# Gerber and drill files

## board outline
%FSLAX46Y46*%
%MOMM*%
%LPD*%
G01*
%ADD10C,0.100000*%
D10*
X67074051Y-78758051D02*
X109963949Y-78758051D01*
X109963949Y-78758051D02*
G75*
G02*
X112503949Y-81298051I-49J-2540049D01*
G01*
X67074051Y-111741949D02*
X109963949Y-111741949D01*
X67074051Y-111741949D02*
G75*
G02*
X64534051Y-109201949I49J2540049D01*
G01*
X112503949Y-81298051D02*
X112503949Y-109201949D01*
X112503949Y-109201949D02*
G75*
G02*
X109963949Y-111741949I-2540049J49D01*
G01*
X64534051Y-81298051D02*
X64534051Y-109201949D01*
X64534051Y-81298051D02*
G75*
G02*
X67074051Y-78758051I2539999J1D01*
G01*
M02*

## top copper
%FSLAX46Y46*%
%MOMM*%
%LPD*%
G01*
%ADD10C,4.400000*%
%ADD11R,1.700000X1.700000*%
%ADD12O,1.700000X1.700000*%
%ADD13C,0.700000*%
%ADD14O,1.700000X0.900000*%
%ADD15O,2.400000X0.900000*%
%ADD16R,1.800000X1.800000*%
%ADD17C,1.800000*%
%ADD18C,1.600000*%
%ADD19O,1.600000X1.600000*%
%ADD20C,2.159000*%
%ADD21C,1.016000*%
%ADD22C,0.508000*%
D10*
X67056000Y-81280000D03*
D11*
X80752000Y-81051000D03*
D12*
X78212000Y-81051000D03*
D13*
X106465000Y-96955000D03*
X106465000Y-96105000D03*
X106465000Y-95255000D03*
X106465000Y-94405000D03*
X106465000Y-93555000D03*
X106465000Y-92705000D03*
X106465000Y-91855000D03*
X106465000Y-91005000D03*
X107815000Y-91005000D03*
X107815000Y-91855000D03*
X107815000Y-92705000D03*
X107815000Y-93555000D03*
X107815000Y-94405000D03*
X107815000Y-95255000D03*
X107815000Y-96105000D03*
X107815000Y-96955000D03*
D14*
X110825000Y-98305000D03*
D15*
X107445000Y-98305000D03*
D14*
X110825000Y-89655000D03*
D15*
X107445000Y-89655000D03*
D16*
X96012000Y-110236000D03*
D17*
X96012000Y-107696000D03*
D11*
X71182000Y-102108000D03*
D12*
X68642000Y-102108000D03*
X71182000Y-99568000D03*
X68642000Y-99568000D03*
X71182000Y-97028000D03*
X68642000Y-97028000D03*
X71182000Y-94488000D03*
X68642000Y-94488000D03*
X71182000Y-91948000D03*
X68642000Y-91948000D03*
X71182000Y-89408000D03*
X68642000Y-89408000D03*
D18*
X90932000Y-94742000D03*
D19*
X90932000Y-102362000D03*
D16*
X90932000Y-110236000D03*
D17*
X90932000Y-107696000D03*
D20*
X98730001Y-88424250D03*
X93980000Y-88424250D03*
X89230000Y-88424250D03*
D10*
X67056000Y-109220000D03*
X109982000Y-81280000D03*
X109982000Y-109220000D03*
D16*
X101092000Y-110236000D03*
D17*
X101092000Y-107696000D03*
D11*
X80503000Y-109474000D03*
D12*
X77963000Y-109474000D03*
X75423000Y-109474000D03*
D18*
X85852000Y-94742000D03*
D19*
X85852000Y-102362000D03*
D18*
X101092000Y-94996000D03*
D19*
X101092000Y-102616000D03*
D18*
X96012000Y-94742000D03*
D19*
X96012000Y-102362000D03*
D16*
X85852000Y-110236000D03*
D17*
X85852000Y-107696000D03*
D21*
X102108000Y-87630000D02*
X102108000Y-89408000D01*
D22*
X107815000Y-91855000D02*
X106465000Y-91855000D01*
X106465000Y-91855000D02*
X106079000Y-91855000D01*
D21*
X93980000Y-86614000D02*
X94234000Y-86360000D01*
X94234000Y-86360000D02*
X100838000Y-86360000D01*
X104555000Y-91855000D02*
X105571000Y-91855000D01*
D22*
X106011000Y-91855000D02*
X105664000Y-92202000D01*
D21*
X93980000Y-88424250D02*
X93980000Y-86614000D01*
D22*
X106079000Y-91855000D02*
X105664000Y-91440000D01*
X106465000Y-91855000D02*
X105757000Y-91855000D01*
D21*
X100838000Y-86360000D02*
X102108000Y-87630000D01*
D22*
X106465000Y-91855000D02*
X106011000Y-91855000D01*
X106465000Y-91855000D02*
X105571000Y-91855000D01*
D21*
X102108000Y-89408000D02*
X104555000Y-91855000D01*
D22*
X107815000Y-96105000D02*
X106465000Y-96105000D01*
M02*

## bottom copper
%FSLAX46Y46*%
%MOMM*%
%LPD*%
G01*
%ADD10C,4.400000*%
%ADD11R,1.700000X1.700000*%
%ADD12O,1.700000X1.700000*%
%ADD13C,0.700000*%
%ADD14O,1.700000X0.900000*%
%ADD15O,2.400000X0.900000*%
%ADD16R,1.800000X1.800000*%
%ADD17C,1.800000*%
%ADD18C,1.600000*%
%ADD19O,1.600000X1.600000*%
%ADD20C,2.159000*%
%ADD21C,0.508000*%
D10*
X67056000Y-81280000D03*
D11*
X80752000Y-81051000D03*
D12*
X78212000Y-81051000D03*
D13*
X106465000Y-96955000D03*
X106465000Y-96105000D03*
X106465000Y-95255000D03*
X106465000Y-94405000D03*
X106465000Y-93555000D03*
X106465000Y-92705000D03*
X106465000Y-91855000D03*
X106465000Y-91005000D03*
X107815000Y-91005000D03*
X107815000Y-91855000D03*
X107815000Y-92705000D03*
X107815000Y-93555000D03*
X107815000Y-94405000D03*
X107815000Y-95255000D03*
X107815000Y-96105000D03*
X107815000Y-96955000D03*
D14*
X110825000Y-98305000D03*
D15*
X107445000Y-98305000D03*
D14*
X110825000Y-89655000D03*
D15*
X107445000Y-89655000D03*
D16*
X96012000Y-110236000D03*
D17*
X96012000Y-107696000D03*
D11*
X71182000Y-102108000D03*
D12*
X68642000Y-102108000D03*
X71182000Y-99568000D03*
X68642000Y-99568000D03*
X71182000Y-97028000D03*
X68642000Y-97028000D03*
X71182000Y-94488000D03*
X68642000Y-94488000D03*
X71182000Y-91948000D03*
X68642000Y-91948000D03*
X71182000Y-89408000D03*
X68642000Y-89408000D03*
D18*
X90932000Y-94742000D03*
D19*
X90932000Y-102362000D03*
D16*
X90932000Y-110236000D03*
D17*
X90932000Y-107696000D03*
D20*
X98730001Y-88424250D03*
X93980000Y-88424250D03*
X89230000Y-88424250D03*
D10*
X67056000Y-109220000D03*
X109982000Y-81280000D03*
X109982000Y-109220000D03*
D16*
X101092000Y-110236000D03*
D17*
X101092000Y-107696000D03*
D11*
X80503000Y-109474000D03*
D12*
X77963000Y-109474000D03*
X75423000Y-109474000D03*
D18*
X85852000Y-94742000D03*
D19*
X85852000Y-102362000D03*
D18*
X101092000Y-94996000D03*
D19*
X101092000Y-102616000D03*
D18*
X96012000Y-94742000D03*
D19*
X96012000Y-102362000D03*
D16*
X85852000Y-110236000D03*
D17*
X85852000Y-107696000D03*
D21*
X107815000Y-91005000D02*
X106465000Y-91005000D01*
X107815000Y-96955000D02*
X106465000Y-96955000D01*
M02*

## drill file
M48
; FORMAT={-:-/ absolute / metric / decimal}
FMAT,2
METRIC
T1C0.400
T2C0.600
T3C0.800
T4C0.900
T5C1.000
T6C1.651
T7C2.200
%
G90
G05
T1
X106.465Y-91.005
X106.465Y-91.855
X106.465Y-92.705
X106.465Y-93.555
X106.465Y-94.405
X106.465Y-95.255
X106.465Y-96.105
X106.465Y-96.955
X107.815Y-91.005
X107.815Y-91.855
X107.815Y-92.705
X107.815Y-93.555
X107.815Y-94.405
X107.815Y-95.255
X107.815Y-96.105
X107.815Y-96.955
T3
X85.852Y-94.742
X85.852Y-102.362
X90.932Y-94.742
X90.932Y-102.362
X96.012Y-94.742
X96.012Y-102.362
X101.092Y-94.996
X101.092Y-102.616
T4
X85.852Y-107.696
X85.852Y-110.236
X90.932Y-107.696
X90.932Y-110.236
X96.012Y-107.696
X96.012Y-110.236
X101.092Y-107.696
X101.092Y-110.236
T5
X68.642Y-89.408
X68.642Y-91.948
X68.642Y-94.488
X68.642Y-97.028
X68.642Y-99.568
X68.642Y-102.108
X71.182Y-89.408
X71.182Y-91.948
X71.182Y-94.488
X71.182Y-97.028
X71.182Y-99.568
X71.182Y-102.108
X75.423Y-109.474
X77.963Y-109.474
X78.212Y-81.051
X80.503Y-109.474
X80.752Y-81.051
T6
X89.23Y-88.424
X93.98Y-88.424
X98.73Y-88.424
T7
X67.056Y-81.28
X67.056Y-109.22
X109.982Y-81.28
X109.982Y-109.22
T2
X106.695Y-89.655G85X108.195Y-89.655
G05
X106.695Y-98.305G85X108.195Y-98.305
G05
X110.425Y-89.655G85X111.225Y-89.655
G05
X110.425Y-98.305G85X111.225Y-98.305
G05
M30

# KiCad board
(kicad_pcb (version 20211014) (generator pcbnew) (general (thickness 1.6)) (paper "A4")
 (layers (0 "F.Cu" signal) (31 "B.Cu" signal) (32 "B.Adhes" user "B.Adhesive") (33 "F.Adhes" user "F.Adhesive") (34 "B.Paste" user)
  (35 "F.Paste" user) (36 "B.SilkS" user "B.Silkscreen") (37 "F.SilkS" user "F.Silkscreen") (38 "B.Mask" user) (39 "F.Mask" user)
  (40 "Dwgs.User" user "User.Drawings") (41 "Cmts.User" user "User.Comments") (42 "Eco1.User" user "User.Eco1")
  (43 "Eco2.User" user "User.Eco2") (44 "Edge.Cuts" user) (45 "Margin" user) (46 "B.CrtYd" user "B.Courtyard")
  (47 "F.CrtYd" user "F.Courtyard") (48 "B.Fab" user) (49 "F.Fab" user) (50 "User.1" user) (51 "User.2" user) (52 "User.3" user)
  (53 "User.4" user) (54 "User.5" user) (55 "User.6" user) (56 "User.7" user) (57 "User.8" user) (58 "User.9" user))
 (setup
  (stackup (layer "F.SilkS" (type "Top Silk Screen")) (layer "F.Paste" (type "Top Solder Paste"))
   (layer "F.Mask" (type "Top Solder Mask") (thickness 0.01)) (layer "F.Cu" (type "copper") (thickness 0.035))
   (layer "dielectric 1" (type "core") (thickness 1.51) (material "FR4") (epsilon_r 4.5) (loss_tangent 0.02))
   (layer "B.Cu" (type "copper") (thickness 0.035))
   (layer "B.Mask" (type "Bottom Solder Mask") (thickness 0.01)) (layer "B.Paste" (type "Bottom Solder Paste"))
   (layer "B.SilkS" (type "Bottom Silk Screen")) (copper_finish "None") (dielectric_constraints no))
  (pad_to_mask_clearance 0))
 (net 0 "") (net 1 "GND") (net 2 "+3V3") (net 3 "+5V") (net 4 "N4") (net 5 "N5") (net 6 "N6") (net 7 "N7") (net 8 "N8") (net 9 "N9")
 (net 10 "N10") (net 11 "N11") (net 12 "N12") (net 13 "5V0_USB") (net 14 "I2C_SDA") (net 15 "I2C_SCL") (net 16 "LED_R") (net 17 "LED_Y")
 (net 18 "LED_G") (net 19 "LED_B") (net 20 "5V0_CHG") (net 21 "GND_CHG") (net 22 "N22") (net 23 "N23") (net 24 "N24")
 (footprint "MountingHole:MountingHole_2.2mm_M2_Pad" (layer "F.Cu") (at 67.056 81.28)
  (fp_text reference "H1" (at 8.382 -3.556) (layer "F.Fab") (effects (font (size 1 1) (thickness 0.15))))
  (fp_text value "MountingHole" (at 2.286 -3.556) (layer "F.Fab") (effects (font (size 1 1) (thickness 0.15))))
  (pad "1" thru_hole circle (at 0 0) (size 4.4 4.4) (drill 2.2) (layers *.Cu *.Mask)))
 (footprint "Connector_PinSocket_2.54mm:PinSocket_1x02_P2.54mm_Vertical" (layer "F.Cu") (at 80.752 81.051 -90)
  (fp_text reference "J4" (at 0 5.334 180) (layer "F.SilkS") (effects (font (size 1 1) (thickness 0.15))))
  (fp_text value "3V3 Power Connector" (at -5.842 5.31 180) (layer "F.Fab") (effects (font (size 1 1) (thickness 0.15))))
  (pad "1" thru_hole rect (at 0 0 270) (size 1.7 1.7) (drill 1) (layers *.Cu *.Mask) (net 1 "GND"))
  (pad "2" thru_hole oval (at 0 2.54 270) (size 1.7 1.7) (drill 1) (layers *.Cu *.Mask) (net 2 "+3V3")))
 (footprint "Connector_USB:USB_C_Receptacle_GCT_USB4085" (layer "F.Cu") (at 106.465 96.955 90)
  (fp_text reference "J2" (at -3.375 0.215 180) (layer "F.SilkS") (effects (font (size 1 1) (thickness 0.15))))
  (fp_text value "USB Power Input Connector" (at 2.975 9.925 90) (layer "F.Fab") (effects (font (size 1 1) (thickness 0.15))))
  (pad "A1" thru_hole circle (at 0 0 90) (size 0.7 0.7) (drill 0.4) (layers *.Cu *.Mask) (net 1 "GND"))
  (pad "A4" thru_hole circle (at 0.85 0 90) (size 0.7 0.7) (drill 0.4) (layers *.Cu *.Mask) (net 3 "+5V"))
  (pad "A5" thru_hole circle (at 1.7 0 90) (size 0.7 0.7) (drill 0.4) (layers *.Cu *.Mask) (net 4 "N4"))
  (pad "A6" thru_hole circle (at 2.55 0 90) (size 0.7 0.7) (drill 0.4) (layers *.Cu *.Mask) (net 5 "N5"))
  (pad "A7" thru_hole circle (at 3.4 0 90) (size 0.7 0.7) (drill 0.4) (layers *.Cu *.Mask) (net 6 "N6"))
  (pad "A8" thru_hole circle (at 4.25 0 90) (size 0.7 0.7) (drill 0.4) (layers *.Cu *.Mask) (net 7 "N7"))
  (pad "A9" thru_hole circle (at 5.1 0 90) (size 0.7 0.7) (drill 0.4) (layers *.Cu *.Mask) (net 3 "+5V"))
  (pad "A12" thru_hole circle (at 5.95 0 90) (size 0.7 0.7) (drill 0.4) (layers *.Cu *.Mask) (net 1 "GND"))
  (pad "B1" thru_hole circle (at 5.95 1.35 90) (size 0.7 0.7) (drill 0.4) (layers *.Cu *.Mask) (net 1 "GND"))
  (pad "B4" thru_hole circle (at 5.1 1.35 90) (size 0.7 0.7) (drill 0.4) (layers *.Cu *.Mask) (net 3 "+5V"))
  (pad "B5" thru_hole circle (at 4.25 1.35 90) (size 0.7 0.7) (drill 0.4) (layers *.Cu *.Mask) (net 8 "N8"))
  (pad "B6" thru_hole circle (at 3.4 1.35 90) (size 0.7 0.7) (drill 0.4) (layers *.Cu *.Mask) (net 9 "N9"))
  (pad "B7" thru_hole circle (at 2.55 1.35 90) (size 0.7 0.7) (drill 0.4) (layers *.Cu *.Mask) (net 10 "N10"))
  (pad "B8" thru_hole circle (at 1.7 1.35 90) (size 0.7 0.7) (drill 0.4) (layers *.Cu *.Mask) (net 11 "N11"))
  (pad "B9" thru_hole circle (at 0.85 1.35 90) (size 0.7 0.7) (drill 0.4) (layers *.Cu *.Mask) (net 3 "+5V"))
  (pad "B12" thru_hole circle (at 0 1.35 90) (size 0.7 0.7) (drill 0.4) (layers *.Cu *.Mask) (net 1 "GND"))
  (pad "S1" thru_hole oval (at -1.35 4.36 90) (size 0.9 1.7) (drill oval 0.6 1.4) (layers *.Cu *.Mask) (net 1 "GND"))
  (pad "S1" thru_hole oval (at -1.35 0.98 90) (size 0.9 2.4) (drill oval 0.6 2.1) (layers *.Cu *.Mask) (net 1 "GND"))
  (pad "S1" thru_hole oval (at 7.3 4.36 90) (size 0.9 1.7) (drill oval 0.6 1.4) (layers *.Cu *.Mask) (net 1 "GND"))
  (pad "S1" thru_hole oval (at 7.3 0.98 90) (size 0.9 2.4) (drill oval 0.6 2.1) (layers *.Cu *.Mask) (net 1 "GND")))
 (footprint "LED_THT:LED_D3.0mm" (layer "F.Cu") (at 96.012 110.236 90)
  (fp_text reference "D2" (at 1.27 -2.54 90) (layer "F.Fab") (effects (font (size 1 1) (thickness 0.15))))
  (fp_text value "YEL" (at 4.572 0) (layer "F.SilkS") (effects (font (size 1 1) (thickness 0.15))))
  (pad "1" thru_hole rect (at 0 0 90) (size 1.8 1.8) (drill 0.9) (layers *.Cu *.Mask) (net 1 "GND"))
  (pad "2" thru_hole circle (at 2.54 0 90) (size 1.8 1.8) (drill 0.9) (layers *.Cu *.Mask) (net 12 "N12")))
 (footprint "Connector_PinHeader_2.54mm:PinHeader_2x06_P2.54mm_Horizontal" (layer "F.Cu") (at 71.182 102.108 180)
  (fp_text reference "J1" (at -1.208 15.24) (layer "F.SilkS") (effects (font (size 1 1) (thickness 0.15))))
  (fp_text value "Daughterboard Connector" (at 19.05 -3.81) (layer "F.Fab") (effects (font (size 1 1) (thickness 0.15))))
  (pad "1" thru_hole rect (at 0 0 180) (size 1.7 1.7) (drill 1) (layers *.Cu *.Mask) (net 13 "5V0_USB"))
  (pad "2" thru_hole oval (at 2.54 0 180) (size 1.7 1.7) (drill 1) (layers *.Cu *.Mask) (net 2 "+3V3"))
  (pad "3" thru_hole oval (at 0 2.54 180) (size 1.7 1.7) (drill 1) (layers *.Cu *.Mask) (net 1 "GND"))
  (pad "4" thru_hole oval (at 2.54 2.54 180) (size 1.7 1.7) (drill 1) (layers *.Cu *.Mask) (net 1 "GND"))
  (pad "5" thru_hole oval (at 0 5.08 180) (size 1.7 1.7) (drill 1) (layers *.Cu *.Mask) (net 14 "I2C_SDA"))
  (pad "6" thru_hole oval (at 2.54 5.08 180) (size 1.7 1.7) (drill 1) (layers *.Cu *.Mask) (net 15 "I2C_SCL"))
  (pad "7" thru_hole oval (at 0 7.62 180) (size 1.7 1.7) (drill 1) (layers *.Cu *.Mask) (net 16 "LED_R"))
  (pad "8" thru_hole oval (at 2.54 7.62 180) (size 1.7 1.7) (drill 1) (layers *.Cu *.Mask) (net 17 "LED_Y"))
  (pad "9" thru_hole oval (at 0 10.16 180) (size 1.7 1.7) (drill 1) (layers *.Cu *.Mask) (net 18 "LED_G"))
  (pad "10" thru_hole oval (at 2.54 10.16 180) (size 1.7 1.7) (drill 1) (layers *.Cu *.Mask) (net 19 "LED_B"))
  (pad "11" thru_hole oval (at 0 12.7 180) (size 1.7 1.7) (drill 1) (layers *.Cu *.Mask) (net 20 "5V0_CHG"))
  (pad "12" thru_hole oval (at 2.54 12.7 180) (size 1.7 1.7) (drill 1) (layers *.Cu *.Mask) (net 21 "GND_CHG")))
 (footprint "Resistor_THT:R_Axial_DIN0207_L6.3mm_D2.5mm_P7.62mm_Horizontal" (layer "F.Cu") (at 90.932 94.742 -90)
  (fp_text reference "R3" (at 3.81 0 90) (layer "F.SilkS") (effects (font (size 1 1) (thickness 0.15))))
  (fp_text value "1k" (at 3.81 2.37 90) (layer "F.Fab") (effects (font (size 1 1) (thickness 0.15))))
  (pad "1" thru_hole circle (at 0 0 270) (size 1.6 1.6) (drill 0.8) (layers *.Cu *.Mask) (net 18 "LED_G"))
  (pad "2" thru_hole oval (at 7.62 0 270) (size 1.6 1.6) (drill 0.8) (layers *.Cu *.Mask) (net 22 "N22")))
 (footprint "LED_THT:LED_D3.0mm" (layer "F.Cu") (at 90.932 110.236 90)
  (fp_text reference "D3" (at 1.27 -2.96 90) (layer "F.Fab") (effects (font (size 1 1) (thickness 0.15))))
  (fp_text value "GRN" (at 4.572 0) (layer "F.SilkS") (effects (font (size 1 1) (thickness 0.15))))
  (pad "1" thru_hole rect (at 0 0 90) (size 1.8 1.8) (drill 0.9) (layers *.Cu *.Mask) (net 1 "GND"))
  (pad "2" thru_hole circle (at 2.54 0 90) (size 1.8 1.8) (drill 0.9) (layers *.Cu *.Mask) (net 22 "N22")))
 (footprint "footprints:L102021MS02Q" (layer "F.Cu") (at 98.730001 88.42425 180)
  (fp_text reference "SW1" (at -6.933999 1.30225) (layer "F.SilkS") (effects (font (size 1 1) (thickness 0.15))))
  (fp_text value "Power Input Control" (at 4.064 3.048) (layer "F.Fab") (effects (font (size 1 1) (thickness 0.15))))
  (pad "1" thru_hole circle locked (at 0 0 180) (size 2.159 2.159) (drill 1.651) (layers *.Cu *.Mask) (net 13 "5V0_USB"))
  (pad "2" thru_hole circle locked (at 4.750001 0 180) (size 2.159 2.159) (drill 1.651) (layers *.Cu *.Mask) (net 3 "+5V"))
  (pad "3" thru_hole circle locked (at 9.500001 0 180) (size 2.159 2.159) (drill 1.651) (layers *.Cu *.Mask) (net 20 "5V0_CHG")))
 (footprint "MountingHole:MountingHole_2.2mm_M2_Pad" (layer "F.Cu") (at 67.056 109.22)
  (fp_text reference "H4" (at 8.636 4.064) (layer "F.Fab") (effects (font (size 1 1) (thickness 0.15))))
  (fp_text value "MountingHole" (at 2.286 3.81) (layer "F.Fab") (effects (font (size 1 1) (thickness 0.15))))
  (pad "1" thru_hole circle (at 0 0) (size 4.4 4.4) (drill 2.2) (layers *.Cu *.Mask)))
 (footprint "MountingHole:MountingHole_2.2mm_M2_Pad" (layer "F.Cu") (at 109.982 81.28)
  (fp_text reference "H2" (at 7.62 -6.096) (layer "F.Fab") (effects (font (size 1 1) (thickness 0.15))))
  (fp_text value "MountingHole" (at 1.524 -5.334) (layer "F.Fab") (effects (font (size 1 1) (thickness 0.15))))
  (pad "1" thru_hole circle (at 0 0) (size 4.4 4.4) (drill 2.2) (layers *.Cu *.Mask)))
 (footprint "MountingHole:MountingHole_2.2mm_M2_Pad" (layer "F.Cu") (at 109.982 109.22)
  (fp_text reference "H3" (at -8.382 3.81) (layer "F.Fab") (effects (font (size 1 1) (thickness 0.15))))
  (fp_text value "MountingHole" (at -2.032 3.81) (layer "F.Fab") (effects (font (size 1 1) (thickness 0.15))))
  (pad "1" thru_hole circle (at 0 0) (size 4.4 4.4) (drill 2.2) (layers *.Cu *.Mask)))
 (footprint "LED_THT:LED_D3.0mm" (layer "F.Cu") (at 101.092 110.236 90)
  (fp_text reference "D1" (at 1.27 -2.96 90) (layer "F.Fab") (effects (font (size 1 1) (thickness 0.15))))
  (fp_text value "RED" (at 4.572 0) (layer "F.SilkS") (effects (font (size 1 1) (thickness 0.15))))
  (pad "1" thru_hole rect (at 0 0 90) (size 1.8 1.8) (drill 0.9) (layers *.Cu *.Mask) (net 1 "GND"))
  (pad "2" thru_hole circle (at 2.54 0 90) (size 1.8 1.8) (drill 0.9) (layers *.Cu *.Mask) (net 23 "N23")))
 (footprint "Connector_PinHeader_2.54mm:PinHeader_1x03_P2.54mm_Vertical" (layer "F.Cu") (at 80.503 109.474 -90)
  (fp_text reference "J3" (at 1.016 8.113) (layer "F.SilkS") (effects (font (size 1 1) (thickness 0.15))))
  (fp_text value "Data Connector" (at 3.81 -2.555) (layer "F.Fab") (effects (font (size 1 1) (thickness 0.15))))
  (pad "1" thru_hole rect (at 0 0 270) (size 1.7 1.7) (drill 1) (layers *.Cu *.Mask) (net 1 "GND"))
  (pad "2" thru_hole oval (at 0 2.54 270) (size 1.7 1.7) (drill 1) (layers *.Cu *.Mask) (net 14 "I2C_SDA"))
  (pad "3" thru_hole oval (at 0 5.08 270) (size 1.7 1.7) (drill 1) (layers *.Cu *.Mask) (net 15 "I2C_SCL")))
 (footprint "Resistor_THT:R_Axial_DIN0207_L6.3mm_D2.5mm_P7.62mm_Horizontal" (layer "F.Cu") (at 85.852 94.742 -90)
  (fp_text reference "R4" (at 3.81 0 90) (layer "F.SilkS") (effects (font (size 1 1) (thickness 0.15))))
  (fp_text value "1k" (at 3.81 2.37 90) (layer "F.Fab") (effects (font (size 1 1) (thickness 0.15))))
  (pad "1" thru_hole circle (at 0 0 270) (size 1.6 1.6) (drill 0.8) (layers *.Cu *.Mask) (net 19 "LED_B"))
  (pad "2" thru_hole oval (at 7.62 0 270) (size 1.6 1.6) (drill 0.8) (layers *.Cu *.Mask) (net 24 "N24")))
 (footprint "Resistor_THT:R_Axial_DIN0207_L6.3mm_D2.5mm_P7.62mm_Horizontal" (layer "F.Cu") (at 101.092 94.996 -90)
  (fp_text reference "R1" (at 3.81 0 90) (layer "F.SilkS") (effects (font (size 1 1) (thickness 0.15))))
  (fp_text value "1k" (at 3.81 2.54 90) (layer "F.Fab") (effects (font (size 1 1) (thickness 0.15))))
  (pad "1" thru_hole circle (at 0 0 270) (size 1.6 1.6) (drill 0.8) (layers *.Cu *.Mask) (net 16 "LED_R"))
  (pad "2" thru_hole oval (at 7.62 0 270) (size 1.6 1.6) (drill 0.8) (layers *.Cu *.Mask) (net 23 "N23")))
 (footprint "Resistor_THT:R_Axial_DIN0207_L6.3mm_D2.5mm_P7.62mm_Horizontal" (layer "F.Cu") (at 96.012 94.742 -90)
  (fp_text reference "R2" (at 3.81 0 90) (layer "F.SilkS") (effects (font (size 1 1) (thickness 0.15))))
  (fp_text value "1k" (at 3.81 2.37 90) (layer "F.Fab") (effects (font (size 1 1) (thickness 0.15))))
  (pad "1" thru_hole circle (at 0 0 270) (size 1.6 1.6) (drill 0.8) (layers *.Cu *.Mask) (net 17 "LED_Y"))
  (pad "2" thru_hole oval (at 7.62 0 270) (size 1.6 1.6) (drill 0.8) (layers *.Cu *.Mask) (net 12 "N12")))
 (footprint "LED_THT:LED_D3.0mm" (layer "F.Cu") (at 85.852 110.236 90)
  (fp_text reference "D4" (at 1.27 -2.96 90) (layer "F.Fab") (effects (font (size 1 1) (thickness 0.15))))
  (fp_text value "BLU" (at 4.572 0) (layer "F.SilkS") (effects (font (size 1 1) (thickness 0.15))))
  (pad "1" thru_hole rect (at 0 0 90) (size 1.8 1.8) (drill 0.9) (layers *.Cu *.Mask) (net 1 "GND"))
  (pad "2" thru_hole circle (at 2.54 0 90) (size 1.8 1.8) (drill 0.9) (layers *.Cu *.Mask) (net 24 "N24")))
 (gr_line (start 67.074051 78.758051) (end 109.963949 78.758051) (layer "Edge.Cuts") (width 0.1))
 (gr_arc (start 109.963949 78.758051) (mid 111.76 79.502) (end 112.503949 81.298051) (layer "Edge.Cuts") (width 0.1))
 (gr_line (start 67.074051 111.741949) (end 109.963949 111.741949) (layer "Edge.Cuts") (width 0.1))
 (gr_arc (start 67.074051 111.741949) (mid 65.278 110.998) (end 64.534051 109.201949) (layer "Edge.Cuts") (width 0.1))
 (gr_line (start 112.503949 81.298051) (end 112.503949 109.201949) (layer "Edge.Cuts") (width 0.1))
 (gr_arc (start 112.503949 109.201949) (mid 111.76 110.998) (end 109.963949 111.741949) (layer "Edge.Cuts") (width 0.1))
 (gr_line (start 64.534051 81.298051) (end 64.534051 109.201949) (layer "Edge.Cuts") (width 0.1))
 (gr_arc (start 64.534051 81.298051) (mid 65.278 79.502) (end 67.074051 78.758051) (layer "Edge.Cuts") (width 0.1))
 (segment (start 102.108 87.63) (end 102.108 89.408) (width 1.016) (layer "F.Cu") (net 3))
 (segment (start 107.815 91.855) (end 106.465 91.855) (width 0.508) (layer "F.Cu") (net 3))
 (segment (start 106.465 91.855) (end 106.079 91.855) (width 0.508) (layer "F.Cu") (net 3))
 (segment (start 93.98 86.614) (end 94.234 86.36) (width 1.016) (layer "F.Cu") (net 3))
 (segment (start 94.234 86.36) (end 100.838 86.36) (width 1.016) (layer "F.Cu") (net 3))
 (segment (start 104.555 91.855) (end 105.571 91.855) (width 1.016) (layer "F.Cu") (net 3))
 (segment (start 106.011 91.855) (end 105.664 92.202) (width 0.508) (layer "F.Cu") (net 3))
 (segment (start 93.98 88.42425) (end 93.98 86.614) (width 1.016) (layer "F.Cu") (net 3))
 (segment (start 106.079 91.855) (end 105.664 91.44) (width 0.508) (layer "F.Cu") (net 3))
 (segment (start 106.465 91.855) (end 105.757 91.855) (width 0.508) (layer "F.Cu") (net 3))
 (segment (start 100.838 86.36) (end 102.108 87.63) (width 1.016) (layer "F.Cu") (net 3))
 (segment (start 106.465 91.855) (end 106.011 91.855) (width 0.508) (layer "F.Cu") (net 3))
 (segment (start 106.465 91.855) (end 105.571 91.855) (width 0.508) (layer "F.Cu") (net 3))
 (segment (start 102.108 89.408) (end 104.555 91.855) (width 1.016) (layer "F.Cu") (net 3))
 (segment (start 107.815 96.105) (end 106.465 96.105) (width 0.508) (layer "F.Cu") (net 3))
 (segment (start 107.815 91.005) (end 106.465 91.005) (width 0.508) (layer "B.Cu") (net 1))
 (segment (start 107.815 96.955) (end 106.465 96.955) (width 0.508) (layer "B.Cu") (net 1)))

